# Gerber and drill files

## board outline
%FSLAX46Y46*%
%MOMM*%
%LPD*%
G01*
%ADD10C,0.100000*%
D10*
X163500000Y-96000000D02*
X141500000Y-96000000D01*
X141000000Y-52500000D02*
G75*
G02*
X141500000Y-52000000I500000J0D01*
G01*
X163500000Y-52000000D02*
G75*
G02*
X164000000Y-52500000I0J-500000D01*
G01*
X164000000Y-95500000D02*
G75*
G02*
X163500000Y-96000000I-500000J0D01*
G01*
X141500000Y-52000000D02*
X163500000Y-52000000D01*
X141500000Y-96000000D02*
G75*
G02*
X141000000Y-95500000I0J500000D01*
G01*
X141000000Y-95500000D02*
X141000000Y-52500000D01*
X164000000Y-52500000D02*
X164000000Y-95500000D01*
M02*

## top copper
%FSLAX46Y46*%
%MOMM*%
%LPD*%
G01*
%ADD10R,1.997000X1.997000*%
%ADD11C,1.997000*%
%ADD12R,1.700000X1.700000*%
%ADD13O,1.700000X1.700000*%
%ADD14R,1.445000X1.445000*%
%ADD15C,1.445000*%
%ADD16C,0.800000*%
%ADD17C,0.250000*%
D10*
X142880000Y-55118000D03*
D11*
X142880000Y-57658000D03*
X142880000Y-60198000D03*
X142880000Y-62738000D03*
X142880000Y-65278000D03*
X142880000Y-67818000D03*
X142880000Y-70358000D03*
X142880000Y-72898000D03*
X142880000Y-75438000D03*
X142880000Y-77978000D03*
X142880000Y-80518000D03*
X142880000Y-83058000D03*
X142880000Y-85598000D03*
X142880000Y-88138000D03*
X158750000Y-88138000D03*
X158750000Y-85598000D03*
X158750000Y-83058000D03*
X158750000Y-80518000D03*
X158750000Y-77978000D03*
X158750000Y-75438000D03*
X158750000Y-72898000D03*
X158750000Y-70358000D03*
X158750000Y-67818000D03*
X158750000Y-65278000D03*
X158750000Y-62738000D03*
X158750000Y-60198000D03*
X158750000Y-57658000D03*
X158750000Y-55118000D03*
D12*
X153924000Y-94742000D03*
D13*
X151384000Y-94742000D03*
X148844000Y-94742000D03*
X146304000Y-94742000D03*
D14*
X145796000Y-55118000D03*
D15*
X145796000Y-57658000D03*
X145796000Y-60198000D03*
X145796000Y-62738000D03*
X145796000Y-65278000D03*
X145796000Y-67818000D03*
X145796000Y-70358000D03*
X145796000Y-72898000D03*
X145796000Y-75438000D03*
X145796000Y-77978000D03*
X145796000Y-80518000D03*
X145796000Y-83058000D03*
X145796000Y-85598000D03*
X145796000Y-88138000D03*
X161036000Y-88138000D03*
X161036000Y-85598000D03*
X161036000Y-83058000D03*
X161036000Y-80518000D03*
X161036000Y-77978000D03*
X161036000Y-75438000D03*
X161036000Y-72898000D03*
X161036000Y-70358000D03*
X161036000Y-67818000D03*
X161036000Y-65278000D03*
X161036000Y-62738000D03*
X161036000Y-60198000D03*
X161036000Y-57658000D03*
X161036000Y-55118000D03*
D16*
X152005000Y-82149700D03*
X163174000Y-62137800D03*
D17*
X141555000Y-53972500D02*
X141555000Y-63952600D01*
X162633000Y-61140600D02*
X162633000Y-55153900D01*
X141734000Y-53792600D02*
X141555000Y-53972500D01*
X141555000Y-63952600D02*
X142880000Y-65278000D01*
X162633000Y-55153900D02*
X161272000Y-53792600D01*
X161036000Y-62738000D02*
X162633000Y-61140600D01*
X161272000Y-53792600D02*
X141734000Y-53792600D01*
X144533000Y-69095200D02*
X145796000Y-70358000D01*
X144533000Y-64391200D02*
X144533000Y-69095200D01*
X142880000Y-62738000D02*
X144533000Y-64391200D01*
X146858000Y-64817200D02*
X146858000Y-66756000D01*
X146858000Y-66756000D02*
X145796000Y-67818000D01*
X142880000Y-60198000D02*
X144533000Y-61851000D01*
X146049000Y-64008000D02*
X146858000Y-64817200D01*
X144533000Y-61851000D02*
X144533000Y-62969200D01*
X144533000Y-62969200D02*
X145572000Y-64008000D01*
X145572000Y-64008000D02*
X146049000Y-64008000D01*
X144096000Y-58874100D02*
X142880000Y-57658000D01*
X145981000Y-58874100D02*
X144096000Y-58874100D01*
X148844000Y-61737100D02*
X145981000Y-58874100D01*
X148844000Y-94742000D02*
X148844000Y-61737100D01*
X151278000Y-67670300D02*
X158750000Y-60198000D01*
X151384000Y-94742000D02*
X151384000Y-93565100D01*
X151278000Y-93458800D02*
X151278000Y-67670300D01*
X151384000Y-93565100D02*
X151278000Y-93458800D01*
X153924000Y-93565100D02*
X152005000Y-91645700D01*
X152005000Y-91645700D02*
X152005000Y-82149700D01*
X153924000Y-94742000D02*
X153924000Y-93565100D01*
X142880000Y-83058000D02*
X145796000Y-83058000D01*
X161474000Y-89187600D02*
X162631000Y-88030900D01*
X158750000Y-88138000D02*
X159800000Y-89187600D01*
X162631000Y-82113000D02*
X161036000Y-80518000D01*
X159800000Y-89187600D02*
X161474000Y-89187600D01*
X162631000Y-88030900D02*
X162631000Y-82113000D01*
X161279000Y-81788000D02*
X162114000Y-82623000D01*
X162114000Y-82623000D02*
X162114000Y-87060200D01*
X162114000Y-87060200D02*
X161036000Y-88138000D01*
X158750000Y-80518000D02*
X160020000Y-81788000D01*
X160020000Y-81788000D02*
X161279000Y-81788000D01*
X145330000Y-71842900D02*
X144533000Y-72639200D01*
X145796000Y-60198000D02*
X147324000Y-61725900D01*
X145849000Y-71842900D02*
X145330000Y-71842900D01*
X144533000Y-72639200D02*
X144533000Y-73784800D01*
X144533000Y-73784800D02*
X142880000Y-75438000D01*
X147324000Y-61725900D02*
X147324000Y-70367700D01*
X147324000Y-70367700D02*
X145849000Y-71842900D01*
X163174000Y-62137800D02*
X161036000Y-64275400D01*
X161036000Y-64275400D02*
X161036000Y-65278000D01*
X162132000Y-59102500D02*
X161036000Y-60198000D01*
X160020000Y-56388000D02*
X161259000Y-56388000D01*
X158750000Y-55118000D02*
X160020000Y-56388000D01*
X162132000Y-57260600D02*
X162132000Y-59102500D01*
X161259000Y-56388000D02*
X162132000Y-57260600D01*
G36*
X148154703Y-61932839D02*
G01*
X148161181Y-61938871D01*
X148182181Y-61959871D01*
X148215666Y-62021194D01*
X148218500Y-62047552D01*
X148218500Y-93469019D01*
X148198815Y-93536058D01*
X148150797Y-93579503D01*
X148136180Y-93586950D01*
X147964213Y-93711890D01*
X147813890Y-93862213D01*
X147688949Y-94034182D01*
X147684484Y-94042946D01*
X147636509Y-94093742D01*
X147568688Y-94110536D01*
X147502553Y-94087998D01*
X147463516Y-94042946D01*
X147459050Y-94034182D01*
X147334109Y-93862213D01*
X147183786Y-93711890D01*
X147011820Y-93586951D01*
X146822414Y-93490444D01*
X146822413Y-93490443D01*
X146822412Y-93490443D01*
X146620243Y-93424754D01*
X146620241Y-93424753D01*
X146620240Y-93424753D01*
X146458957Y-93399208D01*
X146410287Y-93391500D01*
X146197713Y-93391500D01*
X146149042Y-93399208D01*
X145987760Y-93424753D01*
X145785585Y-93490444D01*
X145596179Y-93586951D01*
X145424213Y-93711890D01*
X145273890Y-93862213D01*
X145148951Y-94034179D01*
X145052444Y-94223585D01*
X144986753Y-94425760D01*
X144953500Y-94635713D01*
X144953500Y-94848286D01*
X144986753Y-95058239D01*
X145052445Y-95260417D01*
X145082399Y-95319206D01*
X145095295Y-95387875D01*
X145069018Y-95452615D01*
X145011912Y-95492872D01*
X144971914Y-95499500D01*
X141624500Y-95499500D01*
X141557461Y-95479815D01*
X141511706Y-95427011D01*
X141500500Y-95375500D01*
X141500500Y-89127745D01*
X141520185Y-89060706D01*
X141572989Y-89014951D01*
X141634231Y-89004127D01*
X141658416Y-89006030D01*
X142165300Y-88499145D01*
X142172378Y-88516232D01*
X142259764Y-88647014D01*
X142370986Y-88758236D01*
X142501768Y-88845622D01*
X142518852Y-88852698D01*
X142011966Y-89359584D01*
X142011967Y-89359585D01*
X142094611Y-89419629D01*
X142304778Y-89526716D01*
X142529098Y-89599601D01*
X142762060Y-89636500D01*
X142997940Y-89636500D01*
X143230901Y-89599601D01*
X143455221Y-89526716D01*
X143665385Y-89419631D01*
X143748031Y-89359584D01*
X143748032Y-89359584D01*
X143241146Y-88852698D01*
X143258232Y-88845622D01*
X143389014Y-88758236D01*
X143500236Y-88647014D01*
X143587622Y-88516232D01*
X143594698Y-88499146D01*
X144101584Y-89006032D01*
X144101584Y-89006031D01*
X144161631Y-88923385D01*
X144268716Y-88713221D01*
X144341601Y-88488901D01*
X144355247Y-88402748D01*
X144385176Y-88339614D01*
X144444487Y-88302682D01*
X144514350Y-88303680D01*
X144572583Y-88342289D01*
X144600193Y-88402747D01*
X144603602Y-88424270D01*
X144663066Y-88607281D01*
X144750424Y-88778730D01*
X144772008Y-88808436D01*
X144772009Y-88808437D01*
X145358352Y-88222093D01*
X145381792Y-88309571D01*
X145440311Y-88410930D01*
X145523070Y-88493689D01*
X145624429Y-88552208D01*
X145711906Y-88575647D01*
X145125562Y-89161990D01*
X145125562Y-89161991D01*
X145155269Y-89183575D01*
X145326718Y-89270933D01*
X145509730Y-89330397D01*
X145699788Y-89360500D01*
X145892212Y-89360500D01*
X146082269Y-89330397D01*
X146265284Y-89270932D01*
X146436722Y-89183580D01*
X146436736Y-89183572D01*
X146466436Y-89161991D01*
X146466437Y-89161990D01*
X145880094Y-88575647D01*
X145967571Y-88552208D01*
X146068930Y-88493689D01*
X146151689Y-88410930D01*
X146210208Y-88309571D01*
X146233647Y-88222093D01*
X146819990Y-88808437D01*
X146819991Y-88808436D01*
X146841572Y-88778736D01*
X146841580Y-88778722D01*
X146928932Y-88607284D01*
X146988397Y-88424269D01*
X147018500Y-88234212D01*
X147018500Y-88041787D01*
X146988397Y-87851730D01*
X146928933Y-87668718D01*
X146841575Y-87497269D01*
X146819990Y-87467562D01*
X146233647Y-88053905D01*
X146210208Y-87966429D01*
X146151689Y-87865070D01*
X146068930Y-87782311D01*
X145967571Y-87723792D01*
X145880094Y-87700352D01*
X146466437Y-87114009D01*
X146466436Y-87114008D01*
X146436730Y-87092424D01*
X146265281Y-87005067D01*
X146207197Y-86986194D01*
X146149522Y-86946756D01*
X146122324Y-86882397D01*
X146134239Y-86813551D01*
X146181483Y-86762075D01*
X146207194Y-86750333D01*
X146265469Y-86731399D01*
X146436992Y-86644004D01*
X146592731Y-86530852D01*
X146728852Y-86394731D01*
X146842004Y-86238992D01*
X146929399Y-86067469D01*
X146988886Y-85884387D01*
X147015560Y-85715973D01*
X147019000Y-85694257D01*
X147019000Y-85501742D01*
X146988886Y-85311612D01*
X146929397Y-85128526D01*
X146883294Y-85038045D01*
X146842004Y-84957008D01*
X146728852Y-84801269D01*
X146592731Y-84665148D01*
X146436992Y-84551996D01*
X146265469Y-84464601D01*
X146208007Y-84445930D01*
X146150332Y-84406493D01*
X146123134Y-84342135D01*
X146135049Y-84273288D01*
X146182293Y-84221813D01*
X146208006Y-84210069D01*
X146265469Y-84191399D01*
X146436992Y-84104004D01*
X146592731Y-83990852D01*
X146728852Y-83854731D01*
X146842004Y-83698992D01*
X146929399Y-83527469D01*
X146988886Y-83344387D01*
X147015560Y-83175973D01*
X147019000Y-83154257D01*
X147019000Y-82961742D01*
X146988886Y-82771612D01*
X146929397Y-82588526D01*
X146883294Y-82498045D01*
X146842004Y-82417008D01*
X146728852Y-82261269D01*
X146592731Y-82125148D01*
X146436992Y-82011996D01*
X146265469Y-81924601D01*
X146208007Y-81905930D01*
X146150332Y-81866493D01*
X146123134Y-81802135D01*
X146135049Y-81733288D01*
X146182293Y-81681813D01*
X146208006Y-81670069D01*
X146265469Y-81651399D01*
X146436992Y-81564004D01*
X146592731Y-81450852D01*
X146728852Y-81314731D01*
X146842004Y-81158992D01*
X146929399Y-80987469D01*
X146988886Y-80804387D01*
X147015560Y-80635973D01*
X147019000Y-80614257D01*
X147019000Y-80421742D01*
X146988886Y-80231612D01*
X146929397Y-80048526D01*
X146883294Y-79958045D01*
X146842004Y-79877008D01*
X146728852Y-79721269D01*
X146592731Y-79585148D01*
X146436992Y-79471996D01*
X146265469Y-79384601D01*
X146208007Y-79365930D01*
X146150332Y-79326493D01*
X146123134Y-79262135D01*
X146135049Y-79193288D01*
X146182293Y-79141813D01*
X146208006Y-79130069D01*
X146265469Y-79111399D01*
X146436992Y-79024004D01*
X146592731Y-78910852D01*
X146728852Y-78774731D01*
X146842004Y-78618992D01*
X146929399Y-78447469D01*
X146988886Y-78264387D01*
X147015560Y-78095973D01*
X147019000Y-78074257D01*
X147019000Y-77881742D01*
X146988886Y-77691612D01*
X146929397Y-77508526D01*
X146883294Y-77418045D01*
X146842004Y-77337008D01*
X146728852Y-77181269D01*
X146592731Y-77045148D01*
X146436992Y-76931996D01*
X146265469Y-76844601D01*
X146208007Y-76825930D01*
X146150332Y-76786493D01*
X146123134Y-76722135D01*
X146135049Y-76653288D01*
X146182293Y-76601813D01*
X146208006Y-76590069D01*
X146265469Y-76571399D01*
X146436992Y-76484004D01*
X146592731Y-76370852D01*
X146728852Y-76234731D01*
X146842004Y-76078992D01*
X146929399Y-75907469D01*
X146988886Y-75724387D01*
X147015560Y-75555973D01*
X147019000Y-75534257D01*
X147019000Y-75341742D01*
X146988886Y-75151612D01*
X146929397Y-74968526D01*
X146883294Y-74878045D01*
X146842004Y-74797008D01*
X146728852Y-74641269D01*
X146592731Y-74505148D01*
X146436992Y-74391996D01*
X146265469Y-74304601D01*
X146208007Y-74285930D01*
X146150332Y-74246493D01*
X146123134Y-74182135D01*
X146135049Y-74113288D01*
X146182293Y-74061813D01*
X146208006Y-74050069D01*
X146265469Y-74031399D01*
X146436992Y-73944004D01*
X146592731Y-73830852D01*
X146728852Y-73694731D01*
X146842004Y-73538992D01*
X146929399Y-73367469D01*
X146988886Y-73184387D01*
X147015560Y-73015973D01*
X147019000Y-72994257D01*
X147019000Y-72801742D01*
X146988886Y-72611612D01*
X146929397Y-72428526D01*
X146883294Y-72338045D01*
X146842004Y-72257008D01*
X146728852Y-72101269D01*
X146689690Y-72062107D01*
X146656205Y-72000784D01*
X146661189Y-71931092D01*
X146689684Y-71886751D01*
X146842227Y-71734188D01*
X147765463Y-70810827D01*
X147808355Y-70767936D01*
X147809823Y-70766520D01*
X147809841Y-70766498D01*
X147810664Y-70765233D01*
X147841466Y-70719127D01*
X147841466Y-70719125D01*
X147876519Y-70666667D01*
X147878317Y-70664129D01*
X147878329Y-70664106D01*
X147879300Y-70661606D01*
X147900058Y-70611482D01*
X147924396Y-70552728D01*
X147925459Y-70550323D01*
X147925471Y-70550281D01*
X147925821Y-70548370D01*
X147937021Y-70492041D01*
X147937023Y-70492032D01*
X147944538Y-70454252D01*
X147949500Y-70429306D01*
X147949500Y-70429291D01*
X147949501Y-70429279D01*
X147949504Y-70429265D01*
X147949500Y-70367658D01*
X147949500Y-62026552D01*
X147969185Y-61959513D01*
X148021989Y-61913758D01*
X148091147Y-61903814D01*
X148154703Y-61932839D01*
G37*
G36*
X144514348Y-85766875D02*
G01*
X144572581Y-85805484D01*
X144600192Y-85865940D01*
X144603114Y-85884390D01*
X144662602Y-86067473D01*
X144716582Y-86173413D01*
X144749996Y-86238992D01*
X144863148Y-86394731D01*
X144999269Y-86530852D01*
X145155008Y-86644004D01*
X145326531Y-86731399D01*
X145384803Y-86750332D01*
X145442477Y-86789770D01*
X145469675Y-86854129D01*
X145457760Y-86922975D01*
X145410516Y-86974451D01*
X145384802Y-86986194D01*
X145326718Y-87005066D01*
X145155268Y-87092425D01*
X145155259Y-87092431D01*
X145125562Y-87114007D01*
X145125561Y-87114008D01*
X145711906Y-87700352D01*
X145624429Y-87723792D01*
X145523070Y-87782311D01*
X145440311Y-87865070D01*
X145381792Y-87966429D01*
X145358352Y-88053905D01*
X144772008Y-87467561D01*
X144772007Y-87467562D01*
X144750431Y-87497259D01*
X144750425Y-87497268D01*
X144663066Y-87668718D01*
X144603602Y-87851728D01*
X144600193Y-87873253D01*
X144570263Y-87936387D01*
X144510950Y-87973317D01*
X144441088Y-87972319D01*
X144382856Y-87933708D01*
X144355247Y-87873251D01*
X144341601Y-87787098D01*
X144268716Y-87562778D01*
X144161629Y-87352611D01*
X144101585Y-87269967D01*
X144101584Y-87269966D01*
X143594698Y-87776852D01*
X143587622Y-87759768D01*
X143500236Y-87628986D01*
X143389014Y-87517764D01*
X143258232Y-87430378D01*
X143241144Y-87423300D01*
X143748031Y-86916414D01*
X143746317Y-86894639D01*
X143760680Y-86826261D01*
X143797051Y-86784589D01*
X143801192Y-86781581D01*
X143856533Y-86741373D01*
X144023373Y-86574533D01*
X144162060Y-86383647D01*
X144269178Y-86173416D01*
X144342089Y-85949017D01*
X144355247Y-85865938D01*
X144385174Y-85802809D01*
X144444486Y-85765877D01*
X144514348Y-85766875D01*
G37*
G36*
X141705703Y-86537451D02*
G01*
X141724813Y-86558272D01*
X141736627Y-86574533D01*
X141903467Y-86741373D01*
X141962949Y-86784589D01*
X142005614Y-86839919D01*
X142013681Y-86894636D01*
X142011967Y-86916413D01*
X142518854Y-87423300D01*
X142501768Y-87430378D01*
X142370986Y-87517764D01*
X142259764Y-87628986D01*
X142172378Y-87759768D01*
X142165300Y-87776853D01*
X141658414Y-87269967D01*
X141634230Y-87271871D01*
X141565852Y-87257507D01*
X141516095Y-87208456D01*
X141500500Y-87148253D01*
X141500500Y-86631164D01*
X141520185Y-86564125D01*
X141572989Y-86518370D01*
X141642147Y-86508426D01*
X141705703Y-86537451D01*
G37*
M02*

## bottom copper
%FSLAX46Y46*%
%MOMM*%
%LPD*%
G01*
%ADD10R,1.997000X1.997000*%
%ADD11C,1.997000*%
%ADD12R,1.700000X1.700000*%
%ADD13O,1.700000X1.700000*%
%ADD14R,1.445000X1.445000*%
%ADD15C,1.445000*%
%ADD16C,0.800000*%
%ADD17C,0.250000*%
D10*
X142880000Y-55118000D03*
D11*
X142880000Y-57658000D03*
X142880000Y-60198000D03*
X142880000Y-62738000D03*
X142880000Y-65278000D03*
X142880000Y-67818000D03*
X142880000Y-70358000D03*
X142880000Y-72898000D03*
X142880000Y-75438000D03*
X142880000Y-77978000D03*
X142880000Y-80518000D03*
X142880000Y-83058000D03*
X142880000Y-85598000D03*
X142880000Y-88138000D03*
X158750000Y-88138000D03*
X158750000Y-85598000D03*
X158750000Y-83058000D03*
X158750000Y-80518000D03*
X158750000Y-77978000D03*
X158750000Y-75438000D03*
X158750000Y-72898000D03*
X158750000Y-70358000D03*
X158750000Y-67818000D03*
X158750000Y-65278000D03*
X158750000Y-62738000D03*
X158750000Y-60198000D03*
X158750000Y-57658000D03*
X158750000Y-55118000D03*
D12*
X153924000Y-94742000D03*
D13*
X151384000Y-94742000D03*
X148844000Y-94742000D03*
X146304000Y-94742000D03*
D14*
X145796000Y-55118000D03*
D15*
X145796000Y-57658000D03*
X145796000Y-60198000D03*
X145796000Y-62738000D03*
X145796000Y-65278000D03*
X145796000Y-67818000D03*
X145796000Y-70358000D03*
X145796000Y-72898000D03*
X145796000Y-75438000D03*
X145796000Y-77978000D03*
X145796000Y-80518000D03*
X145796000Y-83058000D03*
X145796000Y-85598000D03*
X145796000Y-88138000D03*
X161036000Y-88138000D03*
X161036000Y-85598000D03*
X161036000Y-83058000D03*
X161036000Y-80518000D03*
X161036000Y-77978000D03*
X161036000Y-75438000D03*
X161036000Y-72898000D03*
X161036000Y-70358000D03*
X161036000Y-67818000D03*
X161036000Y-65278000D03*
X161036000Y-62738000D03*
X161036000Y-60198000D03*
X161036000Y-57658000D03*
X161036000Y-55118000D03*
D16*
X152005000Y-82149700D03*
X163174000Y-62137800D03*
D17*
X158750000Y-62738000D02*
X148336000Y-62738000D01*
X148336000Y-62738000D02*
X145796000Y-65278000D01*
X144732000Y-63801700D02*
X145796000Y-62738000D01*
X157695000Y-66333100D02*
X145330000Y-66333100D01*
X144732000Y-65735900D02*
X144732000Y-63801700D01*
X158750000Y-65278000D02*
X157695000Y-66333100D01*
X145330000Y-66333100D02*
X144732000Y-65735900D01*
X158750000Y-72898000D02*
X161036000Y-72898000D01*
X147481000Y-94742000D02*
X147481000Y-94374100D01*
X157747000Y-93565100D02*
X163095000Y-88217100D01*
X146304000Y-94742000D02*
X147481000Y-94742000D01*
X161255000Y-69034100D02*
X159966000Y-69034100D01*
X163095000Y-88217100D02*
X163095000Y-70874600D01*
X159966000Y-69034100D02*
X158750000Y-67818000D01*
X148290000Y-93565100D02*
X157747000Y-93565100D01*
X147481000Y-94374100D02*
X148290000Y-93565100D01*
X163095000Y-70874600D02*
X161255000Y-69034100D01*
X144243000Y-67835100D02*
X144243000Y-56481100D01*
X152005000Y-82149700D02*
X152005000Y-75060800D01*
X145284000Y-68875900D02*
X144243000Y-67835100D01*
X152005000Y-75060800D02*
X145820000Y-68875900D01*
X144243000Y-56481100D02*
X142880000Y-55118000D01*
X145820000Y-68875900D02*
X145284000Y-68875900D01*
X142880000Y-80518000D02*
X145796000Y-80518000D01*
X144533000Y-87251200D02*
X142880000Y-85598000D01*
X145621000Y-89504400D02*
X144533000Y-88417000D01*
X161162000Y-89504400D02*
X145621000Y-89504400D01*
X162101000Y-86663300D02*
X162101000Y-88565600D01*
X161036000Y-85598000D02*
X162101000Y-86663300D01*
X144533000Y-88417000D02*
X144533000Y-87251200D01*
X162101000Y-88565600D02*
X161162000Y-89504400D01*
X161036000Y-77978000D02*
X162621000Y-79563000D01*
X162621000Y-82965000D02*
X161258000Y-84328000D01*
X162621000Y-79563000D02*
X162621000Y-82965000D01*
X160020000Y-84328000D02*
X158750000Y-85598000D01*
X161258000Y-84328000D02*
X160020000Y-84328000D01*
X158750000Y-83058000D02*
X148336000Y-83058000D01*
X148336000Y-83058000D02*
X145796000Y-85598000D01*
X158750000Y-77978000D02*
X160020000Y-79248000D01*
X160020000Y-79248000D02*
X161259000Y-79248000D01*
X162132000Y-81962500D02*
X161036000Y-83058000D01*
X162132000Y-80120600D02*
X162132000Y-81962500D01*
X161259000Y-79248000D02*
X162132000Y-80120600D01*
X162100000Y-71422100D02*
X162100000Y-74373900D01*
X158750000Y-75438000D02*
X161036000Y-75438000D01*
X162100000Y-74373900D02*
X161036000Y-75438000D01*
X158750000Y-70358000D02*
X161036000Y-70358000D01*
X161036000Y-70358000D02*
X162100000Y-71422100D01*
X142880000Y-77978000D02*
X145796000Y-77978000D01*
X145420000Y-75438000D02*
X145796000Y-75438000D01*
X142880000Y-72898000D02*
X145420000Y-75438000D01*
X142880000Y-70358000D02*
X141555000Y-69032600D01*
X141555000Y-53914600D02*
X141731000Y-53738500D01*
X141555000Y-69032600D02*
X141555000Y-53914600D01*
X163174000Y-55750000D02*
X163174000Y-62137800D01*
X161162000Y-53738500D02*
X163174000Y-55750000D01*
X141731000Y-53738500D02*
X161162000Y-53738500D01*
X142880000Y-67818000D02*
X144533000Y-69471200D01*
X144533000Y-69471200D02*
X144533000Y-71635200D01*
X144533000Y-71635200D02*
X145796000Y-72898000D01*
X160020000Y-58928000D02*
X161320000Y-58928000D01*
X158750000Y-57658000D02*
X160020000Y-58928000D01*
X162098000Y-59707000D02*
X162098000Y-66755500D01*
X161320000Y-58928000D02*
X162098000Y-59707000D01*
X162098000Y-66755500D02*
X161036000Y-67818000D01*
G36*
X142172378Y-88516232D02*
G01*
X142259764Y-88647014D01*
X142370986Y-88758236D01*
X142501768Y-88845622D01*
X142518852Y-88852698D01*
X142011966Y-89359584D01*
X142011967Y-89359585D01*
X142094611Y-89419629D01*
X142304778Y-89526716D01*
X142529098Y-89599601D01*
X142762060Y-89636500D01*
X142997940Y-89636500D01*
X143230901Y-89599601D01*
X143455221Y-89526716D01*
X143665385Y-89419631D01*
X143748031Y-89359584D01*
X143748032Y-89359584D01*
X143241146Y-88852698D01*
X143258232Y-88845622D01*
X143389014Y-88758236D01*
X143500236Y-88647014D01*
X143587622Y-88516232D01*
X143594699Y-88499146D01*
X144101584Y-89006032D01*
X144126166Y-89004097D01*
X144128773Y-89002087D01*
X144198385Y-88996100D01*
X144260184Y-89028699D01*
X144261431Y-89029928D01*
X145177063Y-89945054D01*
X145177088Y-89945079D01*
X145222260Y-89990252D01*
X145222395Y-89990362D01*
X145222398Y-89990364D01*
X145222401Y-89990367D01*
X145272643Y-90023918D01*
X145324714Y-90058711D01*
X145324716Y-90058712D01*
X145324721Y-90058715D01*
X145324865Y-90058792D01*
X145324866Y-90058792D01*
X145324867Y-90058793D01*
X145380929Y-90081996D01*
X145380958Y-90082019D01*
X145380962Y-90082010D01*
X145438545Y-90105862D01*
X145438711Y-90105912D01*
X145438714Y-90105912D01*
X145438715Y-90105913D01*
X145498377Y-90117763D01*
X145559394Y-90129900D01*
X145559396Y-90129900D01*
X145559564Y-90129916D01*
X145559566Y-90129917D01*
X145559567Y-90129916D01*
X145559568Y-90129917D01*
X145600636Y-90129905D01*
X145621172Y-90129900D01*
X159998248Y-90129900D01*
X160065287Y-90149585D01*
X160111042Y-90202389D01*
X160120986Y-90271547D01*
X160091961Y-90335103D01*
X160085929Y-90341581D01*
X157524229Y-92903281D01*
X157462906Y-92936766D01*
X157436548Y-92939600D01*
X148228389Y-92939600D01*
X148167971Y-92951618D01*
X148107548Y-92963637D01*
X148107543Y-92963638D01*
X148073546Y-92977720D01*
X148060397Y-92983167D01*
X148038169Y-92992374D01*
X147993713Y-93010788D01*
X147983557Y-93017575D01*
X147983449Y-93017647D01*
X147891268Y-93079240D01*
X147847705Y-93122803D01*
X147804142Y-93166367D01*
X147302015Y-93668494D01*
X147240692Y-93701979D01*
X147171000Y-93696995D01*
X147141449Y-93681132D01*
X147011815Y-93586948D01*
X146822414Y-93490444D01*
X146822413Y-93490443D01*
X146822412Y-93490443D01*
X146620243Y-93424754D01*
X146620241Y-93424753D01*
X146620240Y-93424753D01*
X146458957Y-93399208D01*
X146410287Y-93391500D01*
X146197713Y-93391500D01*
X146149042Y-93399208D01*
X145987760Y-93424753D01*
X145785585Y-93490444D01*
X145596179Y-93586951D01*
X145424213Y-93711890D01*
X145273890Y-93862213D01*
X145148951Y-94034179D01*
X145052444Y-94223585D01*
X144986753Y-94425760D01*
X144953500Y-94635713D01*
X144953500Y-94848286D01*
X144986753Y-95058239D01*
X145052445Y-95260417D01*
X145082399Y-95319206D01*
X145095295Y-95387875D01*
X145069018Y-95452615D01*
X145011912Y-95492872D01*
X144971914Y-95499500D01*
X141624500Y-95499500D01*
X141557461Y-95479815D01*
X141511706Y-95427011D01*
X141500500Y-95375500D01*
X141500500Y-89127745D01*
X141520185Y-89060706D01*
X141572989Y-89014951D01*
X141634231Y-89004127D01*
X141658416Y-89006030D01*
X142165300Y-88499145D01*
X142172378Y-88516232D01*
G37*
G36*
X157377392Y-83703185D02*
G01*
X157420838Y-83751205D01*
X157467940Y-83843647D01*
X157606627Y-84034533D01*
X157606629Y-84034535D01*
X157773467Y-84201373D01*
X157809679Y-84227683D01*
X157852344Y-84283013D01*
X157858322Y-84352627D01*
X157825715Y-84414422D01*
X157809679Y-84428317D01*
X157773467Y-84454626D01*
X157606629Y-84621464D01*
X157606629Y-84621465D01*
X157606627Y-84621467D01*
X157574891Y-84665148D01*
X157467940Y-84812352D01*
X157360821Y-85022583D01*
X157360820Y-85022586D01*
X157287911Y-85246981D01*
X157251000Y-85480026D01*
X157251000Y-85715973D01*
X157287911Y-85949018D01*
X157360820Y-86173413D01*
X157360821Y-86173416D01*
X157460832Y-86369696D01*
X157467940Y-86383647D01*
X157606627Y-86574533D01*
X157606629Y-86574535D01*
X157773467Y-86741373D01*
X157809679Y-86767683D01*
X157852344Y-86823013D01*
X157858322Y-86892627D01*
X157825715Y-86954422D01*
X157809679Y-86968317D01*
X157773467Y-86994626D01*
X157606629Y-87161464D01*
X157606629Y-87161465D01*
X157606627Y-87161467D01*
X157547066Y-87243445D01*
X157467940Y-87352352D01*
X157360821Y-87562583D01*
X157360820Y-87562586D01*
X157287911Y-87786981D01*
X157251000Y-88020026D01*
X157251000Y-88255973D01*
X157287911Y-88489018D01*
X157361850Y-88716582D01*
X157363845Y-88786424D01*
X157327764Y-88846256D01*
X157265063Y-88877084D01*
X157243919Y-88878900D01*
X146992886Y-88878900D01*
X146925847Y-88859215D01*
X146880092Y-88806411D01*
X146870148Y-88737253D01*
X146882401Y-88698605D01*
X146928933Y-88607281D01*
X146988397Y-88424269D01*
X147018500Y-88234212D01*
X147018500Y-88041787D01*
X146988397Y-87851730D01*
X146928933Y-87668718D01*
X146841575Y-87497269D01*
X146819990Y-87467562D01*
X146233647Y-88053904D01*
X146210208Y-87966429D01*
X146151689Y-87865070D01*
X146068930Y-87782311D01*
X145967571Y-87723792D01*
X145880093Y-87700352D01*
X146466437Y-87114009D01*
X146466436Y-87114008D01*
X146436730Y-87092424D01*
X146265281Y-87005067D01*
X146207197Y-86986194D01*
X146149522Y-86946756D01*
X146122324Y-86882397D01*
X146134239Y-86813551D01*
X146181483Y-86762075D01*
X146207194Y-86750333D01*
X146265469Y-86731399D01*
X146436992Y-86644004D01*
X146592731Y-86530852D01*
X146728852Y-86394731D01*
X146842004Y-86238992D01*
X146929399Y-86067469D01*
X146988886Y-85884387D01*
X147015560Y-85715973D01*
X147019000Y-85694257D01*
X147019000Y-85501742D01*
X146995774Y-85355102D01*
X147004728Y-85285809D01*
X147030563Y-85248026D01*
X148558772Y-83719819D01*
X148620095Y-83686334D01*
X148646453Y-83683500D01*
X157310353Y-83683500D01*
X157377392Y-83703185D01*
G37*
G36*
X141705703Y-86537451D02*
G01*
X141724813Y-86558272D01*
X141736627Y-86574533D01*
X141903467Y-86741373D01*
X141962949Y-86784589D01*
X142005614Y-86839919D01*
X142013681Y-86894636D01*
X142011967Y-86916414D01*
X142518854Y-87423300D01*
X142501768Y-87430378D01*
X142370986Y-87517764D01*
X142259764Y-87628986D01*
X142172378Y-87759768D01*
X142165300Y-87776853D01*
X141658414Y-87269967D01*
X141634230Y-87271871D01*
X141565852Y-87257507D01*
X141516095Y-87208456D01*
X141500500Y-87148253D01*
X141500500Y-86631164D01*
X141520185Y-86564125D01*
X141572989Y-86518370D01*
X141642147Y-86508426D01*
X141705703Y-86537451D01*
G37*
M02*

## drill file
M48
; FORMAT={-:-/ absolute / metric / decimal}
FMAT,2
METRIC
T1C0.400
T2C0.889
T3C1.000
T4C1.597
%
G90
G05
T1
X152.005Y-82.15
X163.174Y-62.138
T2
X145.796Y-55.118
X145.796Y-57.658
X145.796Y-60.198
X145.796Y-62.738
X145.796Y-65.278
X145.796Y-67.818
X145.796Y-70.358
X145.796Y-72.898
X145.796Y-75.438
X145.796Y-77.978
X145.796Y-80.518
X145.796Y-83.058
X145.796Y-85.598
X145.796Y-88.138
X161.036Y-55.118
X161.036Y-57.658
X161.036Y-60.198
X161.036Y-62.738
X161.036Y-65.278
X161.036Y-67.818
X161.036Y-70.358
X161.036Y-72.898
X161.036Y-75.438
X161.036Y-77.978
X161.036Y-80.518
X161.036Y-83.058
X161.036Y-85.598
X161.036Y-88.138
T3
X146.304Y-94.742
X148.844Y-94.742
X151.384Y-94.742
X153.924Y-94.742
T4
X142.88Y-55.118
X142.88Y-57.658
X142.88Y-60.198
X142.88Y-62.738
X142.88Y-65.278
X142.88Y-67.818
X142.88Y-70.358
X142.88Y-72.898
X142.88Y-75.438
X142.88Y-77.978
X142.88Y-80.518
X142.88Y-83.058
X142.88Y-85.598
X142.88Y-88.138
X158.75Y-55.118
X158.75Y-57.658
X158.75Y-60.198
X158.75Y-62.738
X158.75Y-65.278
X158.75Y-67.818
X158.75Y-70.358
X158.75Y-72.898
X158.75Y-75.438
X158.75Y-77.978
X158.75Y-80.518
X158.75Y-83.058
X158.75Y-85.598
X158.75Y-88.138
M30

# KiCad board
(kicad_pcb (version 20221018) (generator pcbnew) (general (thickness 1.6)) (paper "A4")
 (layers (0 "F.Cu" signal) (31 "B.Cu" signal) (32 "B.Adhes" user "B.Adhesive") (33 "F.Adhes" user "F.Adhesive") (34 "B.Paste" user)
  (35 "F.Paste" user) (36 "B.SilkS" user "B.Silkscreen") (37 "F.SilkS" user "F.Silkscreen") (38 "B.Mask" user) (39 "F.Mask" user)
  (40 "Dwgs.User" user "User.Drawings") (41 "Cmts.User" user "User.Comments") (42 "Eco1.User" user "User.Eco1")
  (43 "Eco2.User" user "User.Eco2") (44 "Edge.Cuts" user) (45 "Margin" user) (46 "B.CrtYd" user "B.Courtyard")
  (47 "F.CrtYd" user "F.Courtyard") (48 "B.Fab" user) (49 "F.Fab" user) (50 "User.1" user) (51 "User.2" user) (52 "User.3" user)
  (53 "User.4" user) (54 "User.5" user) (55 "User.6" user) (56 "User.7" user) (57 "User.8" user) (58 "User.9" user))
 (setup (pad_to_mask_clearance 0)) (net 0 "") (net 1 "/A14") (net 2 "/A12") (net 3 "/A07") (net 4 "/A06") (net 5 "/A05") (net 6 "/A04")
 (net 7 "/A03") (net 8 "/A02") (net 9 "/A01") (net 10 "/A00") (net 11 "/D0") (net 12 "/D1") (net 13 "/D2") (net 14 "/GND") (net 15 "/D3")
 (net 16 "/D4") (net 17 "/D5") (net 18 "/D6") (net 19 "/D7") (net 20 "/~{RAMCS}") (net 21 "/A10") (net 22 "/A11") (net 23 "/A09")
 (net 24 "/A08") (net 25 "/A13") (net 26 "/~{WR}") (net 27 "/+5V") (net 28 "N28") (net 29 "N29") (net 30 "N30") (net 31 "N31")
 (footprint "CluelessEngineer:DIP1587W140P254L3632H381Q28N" (layer "F.Cu") (at 150.815 71.628)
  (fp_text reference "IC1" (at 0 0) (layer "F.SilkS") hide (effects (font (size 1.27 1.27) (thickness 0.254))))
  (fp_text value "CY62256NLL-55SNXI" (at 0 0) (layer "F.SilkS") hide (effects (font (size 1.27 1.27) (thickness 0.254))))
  (pad "1" thru_hole rect (at -7.935 -16.51) (size 1.997 1.997) (drill 1.597) (layers "*.Cu" "*.Mask") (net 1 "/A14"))
  (pad "2" thru_hole circle (at -7.935 -13.97) (size 1.997 1.997) (drill 1.597) (layers "*.Cu" "*.Mask") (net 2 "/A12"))
  (pad "3" thru_hole circle (at -7.935 -11.43) (size 1.997 1.997) (drill 1.597) (layers "*.Cu" "*.Mask") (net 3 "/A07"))
  (pad "4" thru_hole circle (at -7.935 -8.89) (size 1.997 1.997) (drill 1.597) (layers "*.Cu" "*.Mask") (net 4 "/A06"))
  (pad "5" thru_hole circle (at -7.935 -6.35) (size 1.997 1.997) (drill 1.597) (layers "*.Cu" "*.Mask") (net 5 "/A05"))
  (pad "6" thru_hole circle (at -7.935 -3.81) (size 1.997 1.997) (drill 1.597) (layers "*.Cu" "*.Mask") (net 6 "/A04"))
  (pad "7" thru_hole circle (at -7.935 -1.27) (size 1.997 1.997) (drill 1.597) (layers "*.Cu" "*.Mask") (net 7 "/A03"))
  (pad "8" thru_hole circle (at -7.935 1.27) (size 1.997 1.997) (drill 1.597) (layers "*.Cu" "*.Mask") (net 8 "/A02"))
  (pad "9" thru_hole circle (at -7.935 3.81) (size 1.997 1.997) (drill 1.597) (layers "*.Cu" "*.Mask") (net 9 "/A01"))
  (pad "10" thru_hole circle (at -7.935 6.35) (size 1.997 1.997) (drill 1.597) (layers "*.Cu" "*.Mask") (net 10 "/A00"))
  (pad "11" thru_hole circle (at -7.935 8.89) (size 1.997 1.997) (drill 1.597) (layers "*.Cu" "*.Mask") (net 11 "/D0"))
  (pad "12" thru_hole circle (at -7.935 11.43) (size 1.997 1.997) (drill 1.597) (layers "*.Cu" "*.Mask") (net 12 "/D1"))
  (pad "13" thru_hole circle (at -7.935 13.97) (size 1.997 1.997) (drill 1.597) (layers "*.Cu" "*.Mask") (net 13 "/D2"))
  (pad "14" thru_hole circle (at -7.935 16.51) (size 1.997 1.997) (drill 1.597) (layers "*.Cu" "*.Mask") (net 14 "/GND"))
  (pad "15" thru_hole circle (at 7.935 16.51) (size 1.997 1.997) (drill 1.597) (layers "*.Cu" "*.Mask") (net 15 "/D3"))
  (pad "16" thru_hole circle (at 7.935 13.97) (size 1.997 1.997) (drill 1.597) (layers "*.Cu" "*.Mask") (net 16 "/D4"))
  (pad "17" thru_hole circle (at 7.935 11.43) (size 1.997 1.997) (drill 1.597) (layers "*.Cu" "*.Mask") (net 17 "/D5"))
  (pad "18" thru_hole circle (at 7.935 8.89) (size 1.997 1.997) (drill 1.597) (layers "*.Cu" "*.Mask") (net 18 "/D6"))
  (pad "19" thru_hole circle (at 7.935 6.35) (size 1.997 1.997) (drill 1.597) (layers "*.Cu" "*.Mask") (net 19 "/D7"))
  (pad "20" thru_hole circle (at 7.935 3.81) (size 1.997 1.997) (drill 1.597) (layers "*.Cu" "*.Mask") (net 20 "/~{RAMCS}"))
  (pad "21" thru_hole circle (at 7.935 1.27) (size 1.997 1.997) (drill 1.597) (layers "*.Cu" "*.Mask") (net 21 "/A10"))
  (pad "22" thru_hole circle (at 7.935 -1.27) (size 1.997 1.997) (drill 1.597) (layers "*.Cu" "*.Mask") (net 20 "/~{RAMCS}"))
  (pad "23" thru_hole circle (at 7.935 -3.81) (size 1.997 1.997) (drill 1.597) (layers "*.Cu" "*.Mask") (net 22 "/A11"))
  (pad "24" thru_hole circle (at 7.935 -6.35) (size 1.997 1.997) (drill 1.597) (layers "*.Cu" "*.Mask") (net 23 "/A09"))
  (pad "25" thru_hole circle (at 7.935 -8.89) (size 1.997 1.997) (drill 1.597) (layers "*.Cu" "*.Mask") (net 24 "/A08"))
  (pad "26" thru_hole circle (at 7.935 -11.43) (size 1.997 1.997) (drill 1.597) (layers "*.Cu" "*.Mask") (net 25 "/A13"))
  (pad "27" thru_hole circle (at 7.935 -13.97) (size 1.997 1.997) (drill 1.597) (layers "*.Cu" "*.Mask") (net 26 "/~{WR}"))
  (pad "28" thru_hole circle (at 7.935 -16.51) (size 1.997 1.997) (drill 1.597) (layers "*.Cu" "*.Mask") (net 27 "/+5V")))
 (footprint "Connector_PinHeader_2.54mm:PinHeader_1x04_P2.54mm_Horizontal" (layer "F.Cu") (at 153.924 94.742 -90)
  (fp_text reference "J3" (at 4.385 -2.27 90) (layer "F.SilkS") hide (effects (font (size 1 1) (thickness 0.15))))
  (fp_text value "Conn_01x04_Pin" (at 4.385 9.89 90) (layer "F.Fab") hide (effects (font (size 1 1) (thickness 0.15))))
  (pad "1" thru_hole rect (at 0 0 270) (size 1.7 1.7) (drill 1) (layers "*.Cu" "*.Mask") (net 1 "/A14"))
  (pad "2" thru_hole oval (at 0 2.54 270) (size 1.7 1.7) (drill 1) (layers "*.Cu" "*.Mask") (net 25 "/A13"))
  (pad "3" thru_hole oval (at 0 5.08 270) (size 1.7 1.7) (drill 1) (layers "*.Cu" "*.Mask") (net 2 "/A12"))
  (pad "4" thru_hole oval (at 0 7.62 270) (size 1.7 1.7) (drill 1) (layers "*.Cu" "*.Mask") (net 22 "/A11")))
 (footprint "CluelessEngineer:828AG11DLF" (layer "F.Cu") (at 145.796 55.118 -90)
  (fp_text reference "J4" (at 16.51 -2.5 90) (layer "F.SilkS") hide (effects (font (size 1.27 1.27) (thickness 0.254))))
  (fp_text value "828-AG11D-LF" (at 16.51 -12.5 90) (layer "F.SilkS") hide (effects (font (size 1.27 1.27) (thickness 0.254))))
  (pad "1" thru_hole rect (at 0 0 270) (size 1.445 1.445) (drill 0.889) (layers "*.Cu" "*.Mask") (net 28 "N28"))
  (pad "2" thru_hole circle (at 2.54 0 270) (size 1.445 1.445) (drill 0.889) (layers "*.Cu" "*.Mask") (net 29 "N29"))
  (pad "3" thru_hole circle (at 5.08 0 270) (size 1.445 1.445) (drill 0.889) (layers "*.Cu" "*.Mask") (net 9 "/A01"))
  (pad "4" thru_hole circle (at 7.62 0 270) (size 1.445 1.445) (drill 0.889) (layers "*.Cu" "*.Mask") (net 23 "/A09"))
  (pad "5" thru_hole circle (at 10.16 0 270) (size 1.445 1.445) (drill 0.889) (layers "*.Cu" "*.Mask") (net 24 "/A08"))
  (pad "6" thru_hole circle (at 12.7 0 270) (size 1.445 1.445) (drill 0.889) (layers "*.Cu" "*.Mask") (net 3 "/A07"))
  (pad "7" thru_hole circle (at 15.24 0 270) (size 1.445 1.445) (drill 0.889) (layers "*.Cu" "*.Mask") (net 4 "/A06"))
  (pad "8" thru_hole circle (at 17.78 0 270) (size 1.445 1.445) (drill 0.889) (layers "*.Cu" "*.Mask") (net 6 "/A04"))
  (pad "9" thru_hole circle (at 20.32 0 270) (size 1.445 1.445) (drill 0.889) (layers "*.Cu" "*.Mask") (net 8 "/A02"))
  (pad "10" thru_hole circle (at 22.86 0 270) (size 1.445 1.445) (drill 0.889) (layers "*.Cu" "*.Mask") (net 10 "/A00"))
  (pad "11" thru_hole circle (at 25.4 0 270) (size 1.445 1.445) (drill 0.889) (layers "*.Cu" "*.Mask") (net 11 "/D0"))
  (pad "12" thru_hole circle (at 27.94 0 270) (size 1.445 1.445) (drill 0.889) (layers "*.Cu" "*.Mask") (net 12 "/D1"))
  (pad "13" thru_hole circle (at 30.48 0 270) (size 1.445 1.445) (drill 0.889) (layers "*.Cu" "*.Mask") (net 17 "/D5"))
  (pad "14" thru_hole circle (at 33.02 0 270) (size 1.445 1.445) (drill 0.889) (layers "*.Cu" "*.Mask") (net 14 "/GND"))
  (pad "15" thru_hole circle (at 33.02 -15.24 270) (size 1.445 1.445) (drill 0.889) (layers "*.Cu" "*.Mask") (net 18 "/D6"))
  (pad "16" thru_hole circle (at 30.48 -15.24 270) (size 1.445 1.445) (drill 0.889) (layers "*.Cu" "*.Mask") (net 13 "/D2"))
  (pad "17" thru_hole circle (at 27.94 -15.24 270) (size 1.445 1.445) (drill 0.889) (layers "*.Cu" "*.Mask") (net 19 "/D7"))
  (pad "18" thru_hole circle (at 25.4 -15.24 270) (size 1.445 1.445) (drill 0.889) (layers "*.Cu" "*.Mask") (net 15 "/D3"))
  (pad "19" thru_hole circle (at 22.86 -15.24 270) (size 1.445 1.445) (drill 0.889) (layers "*.Cu" "*.Mask") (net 16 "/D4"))
  (pad "20" thru_hole circle (at 20.32 -15.24 270) (size 1.445 1.445) (drill 0.889) (layers "*.Cu" "*.Mask") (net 20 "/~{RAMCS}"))
  (pad "21" thru_hole circle (at 17.78 -15.24 270) (size 1.445 1.445) (drill 0.889) (layers "*.Cu" "*.Mask") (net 21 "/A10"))
  (pad "22" thru_hole circle (at 15.24 -15.24 270) (size 1.445 1.445) (drill 0.889) (layers "*.Cu" "*.Mask") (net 20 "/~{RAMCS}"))
  (pad "23" thru_hole circle (at 12.7 -15.24 270) (size 1.445 1.445) (drill 0.889) (layers "*.Cu" "*.Mask") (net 26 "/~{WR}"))
  (pad "24" thru_hole circle (at 10.16 -15.24 270) (size 1.445 1.445) (drill 0.889) (layers "*.Cu" "*.Mask") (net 7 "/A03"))
  (pad "25" thru_hole circle (at 7.62 -15.24 270) (size 1.445 1.445) (drill 0.889) (layers "*.Cu" "*.Mask") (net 5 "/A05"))
  (pad "26" thru_hole circle (at 5.08 -15.24 270) (size 1.445 1.445) (drill 0.889) (layers "*.Cu" "*.Mask") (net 27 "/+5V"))
  (pad "27" thru_hole circle (at 2.54 -15.24 270) (size 1.445 1.445) (drill 0.889) (layers "*.Cu" "*.Mask") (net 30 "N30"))
  (pad "28" thru_hole circle (at 0 -15.24 270) (size 1.445 1.445) (drill 0.889) (layers "*.Cu" "*.Mask") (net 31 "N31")))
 (gr_line (start 163.5 96) (end 141.5 96) (stroke (width 0.1) (type default)) (layer "Edge.Cuts"))
 (gr_arc (start 141 52.5) (mid 141.146447 52.146447) (end 141.5 52) (stroke (width 0.1) (type default)) (layer "Edge.Cuts"))
 (gr_arc (start 163.5 52) (mid 163.853553 52.146447) (end 164 52.5) (stroke (width 0.1) (type default)) (layer "Edge.Cuts"))
 (gr_arc (start 164 95.5) (mid 163.853553 95.853553) (end 163.5 96) (stroke (width 0.1) (type default)) (layer "Edge.Cuts"))
 (gr_line (start 141.5 52) (end 163.5 52) (stroke (width 0.1) (type default)) (layer "Edge.Cuts"))
 (gr_arc (start 141.5 96) (mid 141.146447 95.853553) (end 141 95.5) (stroke (width 0.1) (type default)) (layer "Edge.Cuts"))
 (gr_line (start 141 95.5) (end 141 52.5) (stroke (width 0.1) (type default)) (layer "Edge.Cuts"))
 (gr_line (start 164 52.5) (end 164 95.5) (stroke (width 0.1) (type default)) (layer "Edge.Cuts"))
 (segment (start 141.555 53.9725) (end 141.555 63.9526) (width 0.25) (layer "F.Cu") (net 5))
 (segment (start 162.633 61.1406) (end 162.633 55.1539) (width 0.25) (layer "F.Cu") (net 5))
 (segment (start 141.734 53.7926) (end 141.555 53.9725) (width 0.25) (layer "F.Cu") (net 5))
 (segment (start 141.555 63.9526) (end 142.88 65.278) (width 0.25) (layer "F.Cu") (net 5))
 (segment (start 162.633 55.1539) (end 161.272 53.7926) (width 0.25) (layer "F.Cu") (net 5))
 (segment (start 161.036 62.738) (end 162.633 61.1406) (width 0.25) (layer "F.Cu") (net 5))
 (segment (start 161.272 53.7926) (end 141.734 53.7926) (width 0.25) (layer "F.Cu") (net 5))
 (segment (start 144.533 69.0952) (end 145.796 70.358) (width 0.25) (layer "F.Cu") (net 4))
 (segment (start 144.533 64.3912) (end 144.533 69.0952) (width 0.25) (layer "F.Cu") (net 4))
 (segment (start 142.88 62.738) (end 144.533 64.3912) (width 0.25) (layer "F.Cu") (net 4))
 (segment (start 146.858 64.8172) (end 146.858 66.756) (width 0.25) (layer "F.Cu") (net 3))
 (segment (start 146.858 66.756) (end 145.796 67.818) (width 0.25) (layer "F.Cu") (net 3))
 (segment (start 142.88 60.198) (end 144.533 61.851) (width 0.25) (layer "F.Cu") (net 3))
 (segment (start 146.049 64.008) (end 146.858 64.8172) (width 0.25) (layer "F.Cu") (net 3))
 (segment (start 144.533 61.851) (end 144.533 62.9692) (width 0.25) (layer "F.Cu") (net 3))
 (segment (start 144.533 62.9692) (end 145.572 64.008) (width 0.25) (layer "F.Cu") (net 3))
 (segment (start 145.572 64.008) (end 146.049 64.008) (width 0.25) (layer "F.Cu") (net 3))
 (segment (start 158.75 62.738) (end 148.336 62.738) (width 0.25) (layer "B.Cu") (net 24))
 (segment (start 148.336 62.738) (end 145.796 65.278) (width 0.25) (layer "B.Cu") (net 24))
 (segment (start 144.732 63.8017) (end 145.796 62.738) (width 0.25) (layer "B.Cu") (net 23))
 (segment (start 157.695 66.3331) (end 145.33 66.3331) (width 0.25) (layer "B.Cu") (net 23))
 (segment (start 144.732 65.7359) (end 144.732 63.8017) (width 0.25) (layer "B.Cu") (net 23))
 (segment (start 158.75 65.278) (end 157.695 66.3331) (width 0.25) (layer "B.Cu") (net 23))
 (segment (start 145.33 66.3331) (end 144.732 65.7359) (width 0.25) (layer "B.Cu") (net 23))
 (segment (start 158.75 72.898) (end 161.036 72.898) (width 0.25) (layer "B.Cu") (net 21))
 (segment (start 147.481 94.742) (end 147.481 94.3741) (width 0.25) (layer "B.Cu") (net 22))
 (segment (start 157.747 93.5651) (end 163.095 88.2171) (width 0.25) (layer "B.Cu") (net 22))
 (segment (start 146.304 94.742) (end 147.481 94.742) (width 0.25) (layer "B.Cu") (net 22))
 (segment (start 161.255 69.0341) (end 159.966 69.0341) (width 0.25) (layer "B.Cu") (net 22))
 (segment (start 163.095 88.2171) (end 163.095 70.8746) (width 0.25) (layer "B.Cu") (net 22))
 (segment (start 159.966 69.0341) (end 158.75 67.818) (width 0.25) (layer "B.Cu") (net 22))
 (segment (start 148.29 93.5651) (end 157.747 93.5651) (width 0.25) (layer "B.Cu") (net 22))
 (segment (start 147.481 94.3741) (end 148.29 93.5651) (width 0.25) (layer "B.Cu") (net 22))
 (segment (start 163.095 70.8746) (end 161.255 69.0341) (width 0.25) (layer "B.Cu") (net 22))
 (segment (start 144.096 58.8741) (end 142.88 57.658) (width 0.25) (layer "F.Cu") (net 2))
 (segment (start 145.981 58.8741) (end 144.096 58.8741) (width 0.25) (layer "F.Cu") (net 2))
 (segment (start 148.844 61.7371) (end 145.981 58.8741) (width 0.25) (layer "F.Cu") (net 2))
 (segment (start 148.844 94.742) (end 148.844 61.7371) (width 0.25) (layer "F.Cu") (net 2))
 (segment (start 151.278 67.6703) (end 158.75 60.198) (width 0.25) (layer "F.Cu") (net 25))
 (segment (start 151.384 94.742) (end 151.384 93.5651) (width 0.25) (layer "F.Cu") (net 25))
 (segment (start 151.278 93.4588) (end 151.278 67.6703) (width 0.25) (layer "F.Cu") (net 25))
 (segment (start 151.384 93.5651) (end 151.278 93.4588) (width 0.25) (layer "F.Cu") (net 25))
 (segment (start 153.924 93.5651) (end 152.005 91.6457) (width 0.25) (layer "F.Cu") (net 1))
 (segment (start 152.005 91.6457) (end 152.005 82.1497) (width 0.25) (layer "F.Cu") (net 1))
 (segment (start 153.924 94.742) (end 153.924 93.5651) (width 0.25) (layer "F.Cu") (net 1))
 (via (at 152.005 82.1497) (size 0.8) (drill 0.4) (layers "F.Cu" "B.Cu") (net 1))
 (segment (start 144.243 67.8351) (end 144.243 56.4811) (width 0.25) (layer "B.Cu") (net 1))
 (segment (start 152.005 82.1497) (end 152.005 75.0608) (width 0.25) (layer "B.Cu") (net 1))
 (segment (start 145.284 68.8759) (end 144.243 67.8351) (width 0.25) (layer "B.Cu") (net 1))
 (segment (start 152.005 75.0608) (end 145.82 68.8759) (width 0.25) (layer "B.Cu") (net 1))
 (segment (start 144.243 56.4811) (end 142.88 55.118) (width 0.25) (layer "B.Cu") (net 1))
 (segment (start 145.82 68.8759) (end 145.284 68.8759) (width 0.25) (layer "B.Cu") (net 1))
 (segment (start 142.88 80.518) (end 145.796 80.518) (width 0.25) (layer "B.Cu") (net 11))
 (segment (start 142.88 83.058) (end 145.796 83.058) (width 0.25) (layer "F.Cu") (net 12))
 (segment (start 144.533 87.2512) (end 142.88 85.598) (width 0.25) (layer "B.Cu") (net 13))
 (segment (start 145.621 89.5044) (end 144.533 88.417) (width 0.25) (layer "B.Cu") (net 13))
 (segment (start 161.162 89.5044) (end 145.621 89.5044) (width 0.25) (layer "B.Cu") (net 13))
 (segment (start 162.101 86.6633) (end 162.101 88.5656) (width 0.25) (layer "B.Cu") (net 13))
 (segment (start 161.036 85.598) (end 162.101 86.6633) (width 0.25) (layer "B.Cu") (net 13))
 (segment (start 144.533 88.417) (end 144.533 87.2512) (width 0.25) (layer "B.Cu") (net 13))
 (segment (start 162.101 88.5656) (end 161.162 89.5044) (width 0.25) (layer "B.Cu") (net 13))
 (segment (start 161.474 89.1876) (end 162.631 88.0309) (width 0.25) (layer "F.Cu") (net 15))
 (segment (start 158.75 88.138) (end 159.8 89.1876) (width 0.25) (layer "F.Cu") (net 15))
 (segment (start 162.631 82.113) (end 161.036 80.518) (width 0.25) (layer "F.Cu") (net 15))
 (segment (start 159.8 89.1876) (end 161.474 89.1876) (width 0.25) (layer "F.Cu") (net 15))
 (segment (start 162.631 88.0309) (end 162.631 82.113) (width 0.25) (layer "F.Cu") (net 15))
 (segment (start 161.036 77.978) (end 162.621 79.563) (width 0.25) (layer "B.Cu") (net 16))
 (segment (start 162.621 82.965) (end 161.258 84.328) (width 0.25) (layer "B.Cu") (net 16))
 (segment (start 162.621 79.563) (end 162.621 82.965) (width 0.25) (layer "B.Cu") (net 16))
 (segment (start 160.02 84.328) (end 158.75 85.598) (width 0.25) (layer "B.Cu") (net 16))
 (segment (start 161.258 84.328) (end 160.02 84.328) (width 0.25) (layer "B.Cu") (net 16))
 (segment (start 158.75 83.058) (end 148.336 83.058) (width 0.25) (layer "B.Cu") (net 17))
 (segment (start 148.336 83.058) (end 145.796 85.598) (width 0.25) (layer "B.Cu") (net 17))
 (segment (start 161.279 81.788) (end 162.114 82.623) (width 0.25) (layer "F.Cu") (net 18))
 (segment (start 162.114 82.623) (end 162.114 87.0602) (width 0.25) (layer "F.Cu") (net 18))
 (segment (start 162.114 87.0602) (end 161.036 88.138) (width 0.25) (layer "F.Cu") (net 18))
 (segment (start 158.75 80.518) (end 160.02 81.788) (width 0.25) (layer "F.Cu") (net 18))
 (segment (start 160.02 81.788) (end 161.279 81.788) (width 0.25) (layer "F.Cu") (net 18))
 (segment (start 158.75 77.978) (end 160.02 79.248) (width 0.25) (layer "B.Cu") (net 19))
 (segment (start 160.02 79.248) (end 161.259 79.248) (width 0.25) (layer "B.Cu") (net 19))
 (segment (start 162.132 81.9625) (end 161.036 83.058) (width 0.25) (layer "B.Cu") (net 19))
 (segment (start 162.132 80.1206) (end 162.132 81.9625) (width 0.25) (layer "B.Cu") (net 19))
 (segment (start 161.259 79.248) (end 162.132 80.1206) (width 0.25) (layer "B.Cu") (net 19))
 (segment (start 162.1 71.4221) (end 162.1 74.3739) (width 0.25) (layer "B.Cu") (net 20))
 (segment (start 158.75 75.438) (end 161.036 75.438) (width 0.25) (layer "B.Cu") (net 20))
 (segment (start 162.1 74.3739) (end 161.036 75.438) (width 0.25) (layer "B.Cu") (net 20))
 (segment (start 158.75 70.358) (end 161.036 70.358) (width 0.25) (layer "B.Cu") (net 20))
 (segment (start 161.036 70.358) (end 162.1 71.4221) (width 0.25) (layer "B.Cu") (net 20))
 (segment (start 142.88 77.978) (end 145.796 77.978) (width 0.25) (layer "B.Cu") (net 10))
 (segment (start 145.33 71.8429) (end 144.533 72.6392) (width 0.25) (layer "F.Cu") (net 9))
 (segment (start 145.796 60.198) (end 147.324 61.7259) (width 0.25) (layer "F.Cu") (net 9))
 (segment (start 145.849 71.8429) (end 145.33 71.8429) (width 0.25) (layer "F.Cu") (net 9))
 (segment (start 144.533 72.6392) (end 144.533 73.7848) (width 0.25) (layer "F.Cu") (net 9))
 (segment (start 144.533 73.7848) (end 142.88 75.438) (width 0.25) (layer "F.Cu") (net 9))
 (segment (start 147.324 61.7259) (end 147.324 70.3677) (width 0.25) (layer "F.Cu") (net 9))
 (segment (start 147.324 70.3677) (end 145.849 71.8429) (width 0.25) (layer "F.Cu") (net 9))
 (segment (start 145.42 75.438) (end 145.796 75.438) (width 0.25) (layer "B.Cu") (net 8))
 (segment (start 142.88 72.898) (end 145.42 75.438) (width 0.25) (layer "B.Cu") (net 8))
 (segment (start 163.174 62.1378) (end 161.036 64.2754) (width 0.25) (layer "F.Cu") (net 7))
 (segment (start 161.036 64.2754) (end 161.036 65.278) (width 0.25) (layer "F.Cu") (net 7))
 (via (at 163.174 62.1378) (size 0.8) (drill 0.4) (layers "F.Cu" "B.Cu") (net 7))
 (segment (start 142.88 70.358) (end 141.555 69.0326) (width 0.25) (layer "B.Cu") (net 7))
 (segment (start 141.555 53.9146) (end 141.731 53.7385) (width 0.25) (layer "B.Cu") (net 7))
 (segment (start 141.555 69.0326) (end 141.555 53.9146) (width 0.25) (layer "B.Cu") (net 7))
 (segment (start 163.174 55.75) (end 163.174 62.1378) (width 0.25) (layer "B.Cu") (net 7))
 (segment (start 161.162 53.7385) (end 163.174 55.75) (width 0.25) (layer "B.Cu") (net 7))
 (segment (start 141.731 53.7385) (end 161.162 53.7385) (width 0.25) (layer "B.Cu") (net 7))
 (segment (start 142.88 67.818) (end 144.533 69.4712) (width 0.25) (layer "B.Cu") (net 6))
 (segment (start 144.533 69.4712) (end 144.533 71.6352) (width 0.25) (layer "B.Cu") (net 6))
 (segment (start 144.533 71.6352) (end 145.796 72.898) (width 0.25) (layer "B.Cu") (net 6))
 (segment (start 160.02 58.928) (end 161.32 58.928) (width 0.25) (layer "B.Cu") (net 26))
 (segment (start 158.75 57.658) (end 160.02 58.928) (width 0.25) (layer "B.Cu") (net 26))
 (segment (start 162.098 59.707) (end 162.098 66.7555) (width 0.25) (layer "B.Cu") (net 26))
 (segment (start 161.32 58.928) (end 162.098 59.707) (width 0.25) (layer "B.Cu") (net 26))
 (segment (start 162.098 66.7555) (end 161.036 67.818) (width 0.25) (layer "B.Cu") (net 26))
 (segment (start 162.132 59.1025) (end 161.036 60.198) (width 0.25) (layer "F.Cu") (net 27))
 (segment (start 160.02 56.388) (end 161.259 56.388) (width 0.25) (layer "F.Cu") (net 27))
 (segment (start 158.75 55.118) (end 160.02 56.388) (width 0.25) (layer "F.Cu") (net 27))
 (segment (start 162.132 57.2606) (end 162.132 59.1025) (width 0.25) (layer "F.Cu") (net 27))
 (segment (start 161.259 56.388) (end 162.132 57.2606) (width 0.25) (layer "F.Cu") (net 27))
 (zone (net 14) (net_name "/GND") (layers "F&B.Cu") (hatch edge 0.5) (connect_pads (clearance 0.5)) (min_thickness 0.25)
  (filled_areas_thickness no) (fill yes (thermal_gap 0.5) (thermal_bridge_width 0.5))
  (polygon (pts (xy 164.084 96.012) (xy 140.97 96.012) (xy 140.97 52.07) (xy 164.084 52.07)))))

